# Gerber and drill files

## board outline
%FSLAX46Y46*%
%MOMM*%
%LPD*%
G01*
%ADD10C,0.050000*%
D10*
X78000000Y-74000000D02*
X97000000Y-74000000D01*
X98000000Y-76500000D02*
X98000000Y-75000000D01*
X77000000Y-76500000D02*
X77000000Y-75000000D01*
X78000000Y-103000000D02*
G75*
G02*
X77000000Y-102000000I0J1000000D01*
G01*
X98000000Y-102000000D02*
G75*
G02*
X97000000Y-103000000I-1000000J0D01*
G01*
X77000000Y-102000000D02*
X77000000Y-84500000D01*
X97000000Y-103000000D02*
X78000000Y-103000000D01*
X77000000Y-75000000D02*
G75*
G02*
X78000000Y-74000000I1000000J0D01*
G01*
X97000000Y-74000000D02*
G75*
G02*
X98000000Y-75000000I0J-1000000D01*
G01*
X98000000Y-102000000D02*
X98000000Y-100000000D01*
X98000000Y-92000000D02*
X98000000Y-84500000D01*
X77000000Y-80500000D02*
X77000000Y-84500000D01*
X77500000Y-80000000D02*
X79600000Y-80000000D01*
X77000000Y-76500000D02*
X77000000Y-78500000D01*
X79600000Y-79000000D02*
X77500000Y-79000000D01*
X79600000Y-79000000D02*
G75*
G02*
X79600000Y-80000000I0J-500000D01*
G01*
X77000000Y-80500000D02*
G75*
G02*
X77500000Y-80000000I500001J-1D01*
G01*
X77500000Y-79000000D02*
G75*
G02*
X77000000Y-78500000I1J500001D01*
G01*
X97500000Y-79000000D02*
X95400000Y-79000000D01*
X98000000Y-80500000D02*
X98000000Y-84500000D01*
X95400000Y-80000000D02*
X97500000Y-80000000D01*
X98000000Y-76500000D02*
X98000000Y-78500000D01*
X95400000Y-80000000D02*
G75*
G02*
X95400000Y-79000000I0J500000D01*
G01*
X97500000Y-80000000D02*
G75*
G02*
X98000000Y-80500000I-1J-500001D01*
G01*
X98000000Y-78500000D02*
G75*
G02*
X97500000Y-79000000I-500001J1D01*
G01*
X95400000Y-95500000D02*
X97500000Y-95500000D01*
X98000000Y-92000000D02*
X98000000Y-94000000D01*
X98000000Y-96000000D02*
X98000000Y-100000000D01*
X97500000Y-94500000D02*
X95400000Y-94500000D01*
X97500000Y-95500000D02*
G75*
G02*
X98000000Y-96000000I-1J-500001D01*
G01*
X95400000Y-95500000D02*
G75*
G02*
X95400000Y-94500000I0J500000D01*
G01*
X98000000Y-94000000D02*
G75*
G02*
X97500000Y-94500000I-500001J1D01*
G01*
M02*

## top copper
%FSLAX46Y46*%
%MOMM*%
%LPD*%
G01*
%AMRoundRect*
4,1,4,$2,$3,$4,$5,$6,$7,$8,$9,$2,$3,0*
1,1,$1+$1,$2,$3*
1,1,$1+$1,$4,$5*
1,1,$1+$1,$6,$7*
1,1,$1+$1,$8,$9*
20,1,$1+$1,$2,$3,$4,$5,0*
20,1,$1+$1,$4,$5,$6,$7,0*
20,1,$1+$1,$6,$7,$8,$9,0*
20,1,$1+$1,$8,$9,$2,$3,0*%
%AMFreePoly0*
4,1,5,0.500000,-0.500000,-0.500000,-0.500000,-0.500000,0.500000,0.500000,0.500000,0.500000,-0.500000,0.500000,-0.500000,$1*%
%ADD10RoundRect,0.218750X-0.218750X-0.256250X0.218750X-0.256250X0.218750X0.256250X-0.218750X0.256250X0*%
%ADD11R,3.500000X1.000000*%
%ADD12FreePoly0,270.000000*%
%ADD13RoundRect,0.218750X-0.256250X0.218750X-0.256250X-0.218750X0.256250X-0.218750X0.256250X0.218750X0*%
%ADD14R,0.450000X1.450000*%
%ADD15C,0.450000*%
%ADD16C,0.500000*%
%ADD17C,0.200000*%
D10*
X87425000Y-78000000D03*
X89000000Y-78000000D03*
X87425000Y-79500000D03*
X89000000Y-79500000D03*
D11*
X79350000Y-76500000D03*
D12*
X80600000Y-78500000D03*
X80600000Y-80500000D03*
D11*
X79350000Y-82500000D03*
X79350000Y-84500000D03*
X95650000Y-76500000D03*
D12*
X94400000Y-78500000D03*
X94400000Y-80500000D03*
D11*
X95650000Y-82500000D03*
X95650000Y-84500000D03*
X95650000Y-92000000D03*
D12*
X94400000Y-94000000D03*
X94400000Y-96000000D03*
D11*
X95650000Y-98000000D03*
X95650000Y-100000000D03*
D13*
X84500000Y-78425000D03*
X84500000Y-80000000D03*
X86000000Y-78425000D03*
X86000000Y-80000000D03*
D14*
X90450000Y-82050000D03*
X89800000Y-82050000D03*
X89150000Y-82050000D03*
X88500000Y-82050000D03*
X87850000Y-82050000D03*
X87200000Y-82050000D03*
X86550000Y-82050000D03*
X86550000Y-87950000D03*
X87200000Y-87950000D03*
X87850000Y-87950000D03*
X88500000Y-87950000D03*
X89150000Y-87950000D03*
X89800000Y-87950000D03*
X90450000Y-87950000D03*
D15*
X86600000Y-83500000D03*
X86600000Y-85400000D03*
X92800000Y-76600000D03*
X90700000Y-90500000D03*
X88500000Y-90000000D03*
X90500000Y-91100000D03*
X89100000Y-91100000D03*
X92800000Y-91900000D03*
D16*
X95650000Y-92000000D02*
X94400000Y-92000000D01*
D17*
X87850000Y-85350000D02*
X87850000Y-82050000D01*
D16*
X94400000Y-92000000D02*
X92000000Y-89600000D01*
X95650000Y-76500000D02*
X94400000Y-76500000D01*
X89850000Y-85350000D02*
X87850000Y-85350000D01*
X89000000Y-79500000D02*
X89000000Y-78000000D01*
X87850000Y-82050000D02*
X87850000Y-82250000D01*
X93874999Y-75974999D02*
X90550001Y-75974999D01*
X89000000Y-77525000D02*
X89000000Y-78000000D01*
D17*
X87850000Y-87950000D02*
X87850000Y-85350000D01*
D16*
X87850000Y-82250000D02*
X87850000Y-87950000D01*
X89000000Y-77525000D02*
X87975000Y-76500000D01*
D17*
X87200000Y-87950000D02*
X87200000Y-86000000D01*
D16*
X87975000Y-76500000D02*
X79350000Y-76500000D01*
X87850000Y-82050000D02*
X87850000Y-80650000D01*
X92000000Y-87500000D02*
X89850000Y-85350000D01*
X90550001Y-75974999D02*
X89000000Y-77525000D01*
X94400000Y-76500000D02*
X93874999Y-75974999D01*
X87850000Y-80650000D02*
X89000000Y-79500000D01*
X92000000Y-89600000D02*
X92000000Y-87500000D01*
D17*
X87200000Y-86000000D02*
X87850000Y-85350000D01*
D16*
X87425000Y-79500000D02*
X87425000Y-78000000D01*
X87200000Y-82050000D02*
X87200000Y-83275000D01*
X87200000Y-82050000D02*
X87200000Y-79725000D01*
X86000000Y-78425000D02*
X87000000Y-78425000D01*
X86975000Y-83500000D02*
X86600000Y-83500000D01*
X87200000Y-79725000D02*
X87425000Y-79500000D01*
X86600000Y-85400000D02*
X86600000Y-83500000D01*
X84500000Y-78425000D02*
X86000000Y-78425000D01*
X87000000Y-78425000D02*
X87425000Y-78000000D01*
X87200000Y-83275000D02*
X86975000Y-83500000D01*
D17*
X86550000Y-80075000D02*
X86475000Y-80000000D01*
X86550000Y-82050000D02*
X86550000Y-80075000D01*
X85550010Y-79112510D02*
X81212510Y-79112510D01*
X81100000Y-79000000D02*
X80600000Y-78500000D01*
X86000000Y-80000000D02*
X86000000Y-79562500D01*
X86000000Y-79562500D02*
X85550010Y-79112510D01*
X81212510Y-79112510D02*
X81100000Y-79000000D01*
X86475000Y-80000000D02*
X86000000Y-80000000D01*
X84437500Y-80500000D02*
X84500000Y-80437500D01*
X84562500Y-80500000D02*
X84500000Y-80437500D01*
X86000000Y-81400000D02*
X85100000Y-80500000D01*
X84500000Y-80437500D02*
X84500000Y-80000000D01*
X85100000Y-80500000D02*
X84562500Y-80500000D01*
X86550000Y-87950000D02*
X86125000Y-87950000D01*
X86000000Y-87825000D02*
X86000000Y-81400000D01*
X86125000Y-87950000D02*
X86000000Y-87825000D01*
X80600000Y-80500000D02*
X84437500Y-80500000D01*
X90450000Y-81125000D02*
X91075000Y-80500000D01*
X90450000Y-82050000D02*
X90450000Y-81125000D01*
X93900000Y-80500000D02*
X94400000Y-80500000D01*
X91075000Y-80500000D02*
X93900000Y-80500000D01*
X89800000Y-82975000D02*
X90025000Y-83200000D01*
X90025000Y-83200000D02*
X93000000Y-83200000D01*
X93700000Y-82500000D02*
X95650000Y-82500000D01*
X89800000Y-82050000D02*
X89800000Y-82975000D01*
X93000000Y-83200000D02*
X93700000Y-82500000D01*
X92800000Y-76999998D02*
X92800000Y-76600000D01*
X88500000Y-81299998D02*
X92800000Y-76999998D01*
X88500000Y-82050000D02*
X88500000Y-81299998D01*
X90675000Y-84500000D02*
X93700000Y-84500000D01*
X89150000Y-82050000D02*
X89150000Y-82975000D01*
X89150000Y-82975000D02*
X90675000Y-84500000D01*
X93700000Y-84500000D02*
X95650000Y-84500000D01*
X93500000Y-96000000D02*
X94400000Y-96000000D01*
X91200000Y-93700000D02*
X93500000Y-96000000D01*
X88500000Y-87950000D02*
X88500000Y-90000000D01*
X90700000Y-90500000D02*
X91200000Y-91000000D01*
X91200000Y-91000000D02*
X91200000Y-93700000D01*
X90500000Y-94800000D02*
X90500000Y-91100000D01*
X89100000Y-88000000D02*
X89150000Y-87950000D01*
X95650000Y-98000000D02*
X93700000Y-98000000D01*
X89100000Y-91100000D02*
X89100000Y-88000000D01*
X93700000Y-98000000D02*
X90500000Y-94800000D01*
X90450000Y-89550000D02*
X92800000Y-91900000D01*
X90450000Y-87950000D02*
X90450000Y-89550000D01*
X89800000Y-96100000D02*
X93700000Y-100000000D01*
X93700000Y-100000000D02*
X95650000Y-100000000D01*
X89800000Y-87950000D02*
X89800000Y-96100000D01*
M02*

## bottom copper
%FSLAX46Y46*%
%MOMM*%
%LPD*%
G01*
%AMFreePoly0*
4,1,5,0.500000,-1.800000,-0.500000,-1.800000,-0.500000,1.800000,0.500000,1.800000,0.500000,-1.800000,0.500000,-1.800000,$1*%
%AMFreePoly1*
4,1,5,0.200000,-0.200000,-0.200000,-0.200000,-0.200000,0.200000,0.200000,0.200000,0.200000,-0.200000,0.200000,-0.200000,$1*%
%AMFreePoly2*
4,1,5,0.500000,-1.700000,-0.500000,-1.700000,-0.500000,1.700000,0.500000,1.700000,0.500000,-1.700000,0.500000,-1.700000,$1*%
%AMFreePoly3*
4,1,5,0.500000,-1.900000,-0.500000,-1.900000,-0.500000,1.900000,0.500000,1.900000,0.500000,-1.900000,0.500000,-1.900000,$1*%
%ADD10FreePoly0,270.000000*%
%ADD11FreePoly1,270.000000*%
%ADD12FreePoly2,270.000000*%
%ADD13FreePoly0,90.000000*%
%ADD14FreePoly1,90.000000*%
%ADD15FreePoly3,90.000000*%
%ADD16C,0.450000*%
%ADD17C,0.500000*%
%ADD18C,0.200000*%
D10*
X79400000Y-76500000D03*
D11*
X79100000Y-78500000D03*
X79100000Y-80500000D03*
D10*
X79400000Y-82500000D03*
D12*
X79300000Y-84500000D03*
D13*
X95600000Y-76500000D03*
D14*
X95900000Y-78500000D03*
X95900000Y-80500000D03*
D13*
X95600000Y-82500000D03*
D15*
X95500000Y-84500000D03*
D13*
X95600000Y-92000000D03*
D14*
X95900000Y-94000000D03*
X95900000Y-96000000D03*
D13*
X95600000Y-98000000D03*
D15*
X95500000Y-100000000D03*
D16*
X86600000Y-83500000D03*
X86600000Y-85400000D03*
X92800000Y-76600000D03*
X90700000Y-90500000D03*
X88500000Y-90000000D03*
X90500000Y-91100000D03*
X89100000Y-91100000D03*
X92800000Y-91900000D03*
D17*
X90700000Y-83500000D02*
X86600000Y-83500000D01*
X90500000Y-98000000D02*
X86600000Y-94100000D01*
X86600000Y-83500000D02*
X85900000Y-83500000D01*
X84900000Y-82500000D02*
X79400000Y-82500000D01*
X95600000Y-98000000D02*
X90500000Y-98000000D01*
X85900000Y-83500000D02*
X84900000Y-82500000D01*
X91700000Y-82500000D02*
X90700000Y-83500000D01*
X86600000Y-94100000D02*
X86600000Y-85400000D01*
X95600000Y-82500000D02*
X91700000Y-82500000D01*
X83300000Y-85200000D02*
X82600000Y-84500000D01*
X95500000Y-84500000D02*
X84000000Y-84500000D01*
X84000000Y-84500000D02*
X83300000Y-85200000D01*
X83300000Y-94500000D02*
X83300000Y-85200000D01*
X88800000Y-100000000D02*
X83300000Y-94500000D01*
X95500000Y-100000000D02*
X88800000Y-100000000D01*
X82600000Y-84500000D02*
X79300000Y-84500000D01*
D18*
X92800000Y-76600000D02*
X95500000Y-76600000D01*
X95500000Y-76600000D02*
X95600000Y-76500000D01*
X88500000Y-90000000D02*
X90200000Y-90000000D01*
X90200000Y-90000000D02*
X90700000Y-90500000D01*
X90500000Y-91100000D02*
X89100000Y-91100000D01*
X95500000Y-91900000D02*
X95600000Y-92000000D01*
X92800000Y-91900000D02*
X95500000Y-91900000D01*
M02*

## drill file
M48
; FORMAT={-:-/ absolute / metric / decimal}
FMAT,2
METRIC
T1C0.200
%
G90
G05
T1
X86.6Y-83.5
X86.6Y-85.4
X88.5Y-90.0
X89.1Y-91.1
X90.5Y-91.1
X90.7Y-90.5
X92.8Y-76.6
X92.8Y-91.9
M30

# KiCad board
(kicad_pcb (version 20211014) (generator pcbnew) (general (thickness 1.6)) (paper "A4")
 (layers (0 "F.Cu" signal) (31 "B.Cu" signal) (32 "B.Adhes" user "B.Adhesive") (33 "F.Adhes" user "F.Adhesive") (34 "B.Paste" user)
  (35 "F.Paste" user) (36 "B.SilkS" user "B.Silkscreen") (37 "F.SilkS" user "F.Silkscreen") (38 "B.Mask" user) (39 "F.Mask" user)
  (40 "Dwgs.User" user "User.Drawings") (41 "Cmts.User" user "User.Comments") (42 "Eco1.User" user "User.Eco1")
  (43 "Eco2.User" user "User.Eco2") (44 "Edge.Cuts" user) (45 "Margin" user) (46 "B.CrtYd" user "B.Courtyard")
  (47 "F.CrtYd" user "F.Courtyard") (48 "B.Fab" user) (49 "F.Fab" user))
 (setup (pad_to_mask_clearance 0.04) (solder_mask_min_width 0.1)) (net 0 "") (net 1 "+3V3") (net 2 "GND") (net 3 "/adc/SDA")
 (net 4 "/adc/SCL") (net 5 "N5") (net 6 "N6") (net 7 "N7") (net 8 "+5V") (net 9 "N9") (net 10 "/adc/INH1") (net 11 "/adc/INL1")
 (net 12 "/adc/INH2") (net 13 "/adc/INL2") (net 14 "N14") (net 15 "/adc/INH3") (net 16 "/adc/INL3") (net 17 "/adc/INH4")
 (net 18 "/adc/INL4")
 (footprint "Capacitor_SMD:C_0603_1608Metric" (layer "F.Cu") (at 88.2125 78)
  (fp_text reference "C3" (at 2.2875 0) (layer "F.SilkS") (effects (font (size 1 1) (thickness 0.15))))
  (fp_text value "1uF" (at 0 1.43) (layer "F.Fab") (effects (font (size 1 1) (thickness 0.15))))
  (pad "1" smd roundrect locked (at -0.7875 0) (size 0.875 0.95) (layers "F.Cu" "F.Paste" "F.Mask") (roundrect_rratio 0.25) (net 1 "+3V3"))
  (pad "2" smd roundrect locked (at 0.7875 0) (size 0.875 0.95) (layers "F.Cu" "F.Paste" "F.Mask") (roundrect_rratio 0.25) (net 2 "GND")))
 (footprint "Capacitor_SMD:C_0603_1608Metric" (layer "F.Cu") (at 88.2125 79.5)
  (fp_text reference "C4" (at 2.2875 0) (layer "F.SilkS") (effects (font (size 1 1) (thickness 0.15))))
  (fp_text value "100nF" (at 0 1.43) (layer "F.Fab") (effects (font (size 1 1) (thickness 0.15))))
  (pad "1" smd roundrect locked (at -0.7875 0) (size 0.875 0.95) (layers "F.Cu" "F.Paste" "F.Mask") (roundrect_rratio 0.25) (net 1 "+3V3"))
  (pad "2" smd roundrect locked (at 0.7875 0) (size 0.875 0.95) (layers "F.Cu" "F.Paste" "F.Mask") (roundrect_rratio 0.25) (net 2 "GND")))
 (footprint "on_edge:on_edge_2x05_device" (layer "F.Cu") (at 77 80.5 -90)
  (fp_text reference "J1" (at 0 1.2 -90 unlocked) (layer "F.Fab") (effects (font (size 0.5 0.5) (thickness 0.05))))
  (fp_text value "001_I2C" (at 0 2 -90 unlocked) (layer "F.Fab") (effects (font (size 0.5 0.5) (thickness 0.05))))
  (fp_line (start 0 0) (end 4 0) (layer "Edge.Cuts") (width 0.05))
  (fp_line (start -0.5 -0.5) (end -0.5 -2.6) (layer "Edge.Cuts") (width 0.05))
  (fp_line (start -4 0) (end -2 0) (layer "Edge.Cuts") (width 0.05))
  (fp_line (start -1.5 -2.6) (end -1.5 -0.5) (layer "Edge.Cuts") (width 0.05))
  (fp_arc (start -1.5 -2.6) (mid -1 -3.1) (end -0.5 -2.6) (layer "Edge.Cuts") (width 0.05))
  (fp_arc (start 0 0) (mid -0.353553 -0.146447) (end -0.5 -0.5) (layer "Edge.Cuts") (width 0.05))
  (fp_arc (start -1.5 -0.5) (mid -1.646447 -0.146447) (end -2 0) (layer "Edge.Cuts") (width 0.05))
  (pad "1" smd rect locked (at -4 -2.35 90) (size 1 3.5) (layers "F.Cu" "F.Mask") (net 2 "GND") (zone_connect 0))
  (pad "2" smd custom locked (at -2 -3.6 270) (size 1 1) (layers "F.Cu" "F.Mask") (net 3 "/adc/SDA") (zone_connect 0)
   (options (clearance outline) (anchor rect)) (primitives))
  (pad "3" smd custom locked (at 0 -3.6 270) (size 1 1) (layers "F.Cu" "F.Mask") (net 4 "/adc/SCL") (zone_connect 0)
   (options (clearance outline) (anchor rect)) (primitives))
  (pad "4" smd rect locked (at 2 -2.35 90) (size 1 3.5) (layers "F.Cu" "F.Mask") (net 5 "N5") (zone_connect 0))
  (pad "5" smd rect locked (at 4 -2.35 90) (size 1 3.5) (layers "F.Cu" "F.Mask") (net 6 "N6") (zone_connect 0))
  (pad "6" smd custom locked (at -4 -2.4 270) (size 1 3.6) (layers "B.Cu" "B.Mask") (zone_connect 0)
   (options (clearance outline) (anchor rect)) (primitives))
  (pad "7" smd custom locked (at -2 -2.1 270) (size 0.4 0.4) (layers "B.Cu" "B.Mask") (zone_connect 0)
   (options (clearance outline) (anchor rect)) (primitives))
  (pad "8" smd custom locked (at 0 -2.1 270) (size 0.4 0.4) (layers "B.Cu" "B.Mask") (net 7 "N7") (zone_connect 0)
   (options (clearance outline) (anchor rect)) (primitives))
  (pad "9" smd custom locked (at 2 -2.4 270) (size 1 3.6) (layers "B.Cu" "B.Mask") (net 1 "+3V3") (zone_connect 0)
   (options (clearance outline) (anchor rect)) (primitives))
  (pad "10" smd custom locked (at 4 -2.3 270) (size 1 3.4) (layers "B.Cu" "B.Mask") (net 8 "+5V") (zone_connect 0)
   (options (clearance outline) (anchor rect)) (primitives)))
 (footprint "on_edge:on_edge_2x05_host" (layer "F.Cu") (at 98 80.5 -90)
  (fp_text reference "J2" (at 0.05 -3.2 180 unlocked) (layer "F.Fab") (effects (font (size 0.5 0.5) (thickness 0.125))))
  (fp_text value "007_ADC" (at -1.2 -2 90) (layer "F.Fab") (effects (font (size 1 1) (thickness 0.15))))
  (fp_line (start -1.5 0.5) (end -1.5 2.6) (layer "Edge.Cuts") (width 0.05))
  (fp_line (start 0 0) (end 4 0) (layer "Edge.Cuts") (width 0.05))
  (fp_line (start -0.5 2.6) (end -0.5 0.5) (layer "Edge.Cuts") (width 0.05))
  (fp_line (start -4 0) (end -2 0) (layer "Edge.Cuts") (width 0.05))
  (fp_arc (start -0.5 2.6) (mid -1 3.1) (end -1.5 2.6) (layer "Edge.Cuts") (width 0.05))
  (fp_arc (start -0.5 0.5) (mid -0.353553 0.146447) (end 0 0) (layer "Edge.Cuts") (width 0.05))
  (fp_arc (start -2 0) (mid -1.646447 0.146447) (end -1.5 0.5) (layer "Edge.Cuts") (width 0.05))
  (pad "1" smd rect locked (at -4 2.35 270) (size 1 3.5) (layers "F.Cu" "F.Mask") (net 2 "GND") (zone_connect 0))
  (pad "2" smd custom locked (at -2 3.6 270) (size 1 1) (layers "F.Cu" "F.Mask") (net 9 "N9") (zone_connect 0)
   (options (clearance outline) (anchor rect)) (primitives))
  (pad "3" smd custom locked (at 0 3.6 270) (size 1 1) (layers "F.Cu" "F.Mask") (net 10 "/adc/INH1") (zone_connect 0)
   (options (clearance outline) (anchor rect)) (primitives))
  (pad "4" smd rect locked (at 2 2.35 270) (size 1 3.5) (layers "F.Cu" "F.Mask") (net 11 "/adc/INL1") (zone_connect 0))
  (pad "5" smd rect locked (at 4 2.35 270) (size 1 3.5) (layers "F.Cu" "F.Mask") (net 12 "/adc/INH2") (zone_connect 0))
  (pad "6" smd custom locked (at -4 2.4 90) (size 1 3.6) (layers "B.Cu" "B.Mask") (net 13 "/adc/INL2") (zone_connect 0)
   (options (clearance outline) (anchor rect)) (primitives))
  (pad "7" smd custom locked (at -2 2.1 90) (size 0.4 0.4) (layers "B.Cu" "B.Mask") (zone_connect 0)
   (options (clearance outline) (anchor rect)) (primitives))
  (pad "8" smd custom locked (at 0 2.1 90) (size 0.4 0.4) (layers "B.Cu" "B.Mask") (zone_connect 0)
   (options (clearance outline) (anchor rect)) (primitives))
  (pad "9" smd custom locked (at 2 2.4 90) (size 1 3.6) (layers "B.Cu" "B.Mask") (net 1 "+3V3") (zone_connect 0)
   (options (clearance outline) (anchor rect)) (primitives))
  (pad "10" smd custom locked (at 4 2.5 90) (size 1 3.8) (layers "B.Cu" "B.Mask") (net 8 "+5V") (zone_connect 0)
   (options (clearance outline) (anchor rect)) (primitives)))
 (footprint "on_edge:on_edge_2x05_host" (layer "F.Cu") (at 98 96 -90)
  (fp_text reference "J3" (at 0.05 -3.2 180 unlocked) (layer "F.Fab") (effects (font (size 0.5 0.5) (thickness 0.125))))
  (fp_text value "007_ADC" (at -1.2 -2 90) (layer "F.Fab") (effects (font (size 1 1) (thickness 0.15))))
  (fp_line (start -0.5 2.6) (end -0.5 0.5) (layer "Edge.Cuts") (width 0.05))
  (fp_line (start -4 0) (end -2 0) (layer "Edge.Cuts") (width 0.05))
  (fp_line (start 0 0) (end 4 0) (layer "Edge.Cuts") (width 0.05))
  (fp_line (start -1.5 0.5) (end -1.5 2.6) (layer "Edge.Cuts") (width 0.05))
  (fp_arc (start -0.5 0.5) (mid -0.353553 0.146447) (end 0 0) (layer "Edge.Cuts") (width 0.05))
  (fp_arc (start -0.5 2.6) (mid -1 3.1) (end -1.5 2.6) (layer "Edge.Cuts") (width 0.05))
  (fp_arc (start -2 0) (mid -1.646447 0.146447) (end -1.5 0.5) (layer "Edge.Cuts") (width 0.05))
  (pad "1" smd rect locked (at -4 2.35 270) (size 1 3.5) (layers "F.Cu" "F.Mask") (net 2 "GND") (zone_connect 0))
  (pad "2" smd custom locked (at -2 3.6 270) (size 1 1) (layers "F.Cu" "F.Mask") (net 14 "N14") (zone_connect 0)
   (options (clearance outline) (anchor rect)) (primitives))
  (pad "3" smd custom locked (at 0 3.6 270) (size 1 1) (layers "F.Cu" "F.Mask") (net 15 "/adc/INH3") (zone_connect 0)
   (options (clearance outline) (anchor rect)) (primitives))
  (pad "4" smd rect locked (at 2 2.35 270) (size 1 3.5) (layers "F.Cu" "F.Mask") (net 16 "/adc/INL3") (zone_connect 0))
  (pad "5" smd rect locked (at 4 2.35 270) (size 1 3.5) (layers "F.Cu" "F.Mask") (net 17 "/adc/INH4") (zone_connect 0))
  (pad "6" smd custom locked (at -4 2.4 90) (size 1 3.6) (layers "B.Cu" "B.Mask") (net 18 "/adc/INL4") (zone_connect 0)
   (options (clearance outline) (anchor rect)) (primitives))
  (pad "7" smd custom locked (at -2 2.1 90) (size 0.4 0.4) (layers "B.Cu" "B.Mask") (zone_connect 0)
   (options (clearance outline) (anchor rect)) (primitives))
  (pad "8" smd custom locked (at 0 2.1 90) (size 0.4 0.4) (layers "B.Cu" "B.Mask") (zone_connect 0)
   (options (clearance outline) (anchor rect)) (primitives))
  (pad "9" smd custom locked (at 2 2.4 90) (size 1 3.6) (layers "B.Cu" "B.Mask") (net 1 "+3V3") (zone_connect 0)
   (options (clearance outline) (anchor rect)) (primitives))
  (pad "10" smd custom locked (at 4 2.5 90) (size 1 3.8) (layers "B.Cu" "B.Mask") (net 8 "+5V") (zone_connect 0)
   (options (clearance outline) (anchor rect)) (primitives)))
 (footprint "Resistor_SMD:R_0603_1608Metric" (layer "F.Cu") (at 84.5 79.2125 -90)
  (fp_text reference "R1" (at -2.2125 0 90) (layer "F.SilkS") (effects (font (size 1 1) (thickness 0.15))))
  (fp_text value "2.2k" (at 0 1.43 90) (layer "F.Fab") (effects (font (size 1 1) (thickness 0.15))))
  (pad "1" smd roundrect locked (at -0.7875 0 270) (size 0.875 0.95) (layers "F.Cu" "F.Paste" "F.Mask") (roundrect_rratio 0.25)
   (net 1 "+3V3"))
  (pad "2" smd roundrect locked (at 0.7875 0 270) (size 0.875 0.95) (layers "F.Cu" "F.Paste" "F.Mask") (roundrect_rratio 0.25)
   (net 4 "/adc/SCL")))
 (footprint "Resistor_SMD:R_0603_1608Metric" (layer "F.Cu") (at 86 79.2125 -90)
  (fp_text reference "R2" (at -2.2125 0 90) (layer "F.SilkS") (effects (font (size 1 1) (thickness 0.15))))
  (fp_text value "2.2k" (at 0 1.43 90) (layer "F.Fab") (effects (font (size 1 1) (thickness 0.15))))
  (pad "1" smd roundrect locked (at -0.7875 0 270) (size 0.875 0.95) (layers "F.Cu" "F.Paste" "F.Mask") (roundrect_rratio 0.25)
   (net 1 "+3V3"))
  (pad "2" smd roundrect locked (at 0.7875 0 270) (size 0.875 0.95) (layers "F.Cu" "F.Paste" "F.Mask") (roundrect_rratio 0.25)
   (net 3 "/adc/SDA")))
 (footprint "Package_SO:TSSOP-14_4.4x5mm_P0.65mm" (layer "F.Cu") (at 88.5 85 -90)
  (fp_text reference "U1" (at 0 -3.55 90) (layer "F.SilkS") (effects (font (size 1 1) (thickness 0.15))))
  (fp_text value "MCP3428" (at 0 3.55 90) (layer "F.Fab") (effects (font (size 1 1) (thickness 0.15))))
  (pad "1" smd rect locked (at -2.95 -1.95 270) (size 1.45 0.45) (layers "F.Cu" "F.Paste" "F.Mask") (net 10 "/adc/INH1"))
  (pad "2" smd rect locked (at -2.95 -1.3 270) (size 1.45 0.45) (layers "F.Cu" "F.Paste" "F.Mask") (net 11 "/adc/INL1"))
  (pad "3" smd rect locked (at -2.95 -0.65 270) (size 1.45 0.45) (layers "F.Cu" "F.Paste" "F.Mask") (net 12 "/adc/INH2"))
  (pad "4" smd rect locked (at -2.95 0 270) (size 1.45 0.45) (layers "F.Cu" "F.Paste" "F.Mask") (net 13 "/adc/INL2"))
  (pad "5" smd rect locked (at -2.95 0.65 270) (size 1.45 0.45) (layers "F.Cu" "F.Paste" "F.Mask") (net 2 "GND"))
  (pad "6" smd rect locked (at -2.95 1.3 270) (size 1.45 0.45) (layers "F.Cu" "F.Paste" "F.Mask") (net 1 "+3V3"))
  (pad "7" smd rect locked (at -2.95 1.95 270) (size 1.45 0.45) (layers "F.Cu" "F.Paste" "F.Mask") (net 3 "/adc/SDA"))
  (pad "8" smd rect locked (at 2.95 1.95 270) (size 1.45 0.45) (layers "F.Cu" "F.Paste" "F.Mask") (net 4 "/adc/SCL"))
  (pad "9" smd rect locked (at 2.95 1.3 270) (size 1.45 0.45) (layers "F.Cu" "F.Paste" "F.Mask") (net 2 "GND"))
  (pad "10" smd rect locked (at 2.95 0.65 270) (size 1.45 0.45) (layers "F.Cu" "F.Paste" "F.Mask") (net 2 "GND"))
  (pad "11" smd rect locked (at 2.95 0 270) (size 1.45 0.45) (layers "F.Cu" "F.Paste" "F.Mask") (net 15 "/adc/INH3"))
  (pad "12" smd rect locked (at 2.95 -0.65 270) (size 1.45 0.45) (layers "F.Cu" "F.Paste" "F.Mask") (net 16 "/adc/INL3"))
  (pad "13" smd rect locked (at 2.95 -1.3 270) (size 1.45 0.45) (layers "F.Cu" "F.Paste" "F.Mask") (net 17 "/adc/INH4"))
  (pad "14" smd rect locked (at 2.95 -1.95 270) (size 1.45 0.45) (layers "F.Cu" "F.Paste" "F.Mask") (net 18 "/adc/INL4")))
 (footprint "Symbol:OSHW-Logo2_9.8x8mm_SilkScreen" (layer "F.Cu") (at 82.6 93.6)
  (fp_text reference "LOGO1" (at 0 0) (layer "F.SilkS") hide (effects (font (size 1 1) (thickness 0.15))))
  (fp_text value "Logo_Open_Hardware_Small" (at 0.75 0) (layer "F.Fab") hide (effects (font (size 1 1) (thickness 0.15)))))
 (gr_line (start 78 74) (end 97 74) (layer "Edge.Cuts") (width 0.05))
 (gr_line (start 98 76.5) (end 98 75) (layer "Edge.Cuts") (width 0.05))
 (gr_line (start 77 76.5) (end 77 75) (layer "Edge.Cuts") (width 0.05))
 (gr_arc (start 78 103) (mid 77.292893 102.707107) (end 77 102) (layer "Edge.Cuts") (width 0.05))
 (gr_arc (start 98 102) (mid 97.707107 102.707107) (end 97 103) (layer "Edge.Cuts") (width 0.05))
 (gr_line (start 77 102) (end 77 84.5) (layer "Edge.Cuts") (width 0.05))
 (gr_line (start 97 103) (end 78 103) (layer "Edge.Cuts") (width 0.05))
 (gr_arc (start 77 75) (mid 77.292893 74.292893) (end 78 74) (layer "Edge.Cuts") (width 0.05))
 (gr_arc (start 97 74) (mid 97.707107 74.292893) (end 98 75) (layer "Edge.Cuts") (width 0.05))
 (gr_line (start 98 102) (end 98 100) (layer "Edge.Cuts") (width 0.05))
 (gr_line (start 98 92) (end 98 84.5) (layer "Edge.Cuts") (width 0.05))
 (segment (start 95.65 92) (end 94.4 92) (width 0.5) (layer "F.Cu") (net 2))
 (segment (start 87.85 85.35) (end 87.85 82.05) (width 0.2) (layer "F.Cu") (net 2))
 (segment (start 94.4 92) (end 92 89.6) (width 0.5) (layer "F.Cu") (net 2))
 (segment (start 95.65 76.5) (end 94.4 76.5) (width 0.5) (layer "F.Cu") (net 2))
 (segment (start 89.85 85.35) (end 87.85 85.35) (width 0.5) (layer "F.Cu") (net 2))
 (segment (start 89 79.5) (end 89 78) (width 0.5) (layer "F.Cu") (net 2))
 (segment (start 87.85 82.05) (end 87.85 82.25) (width 0.5) (layer "F.Cu") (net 2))
 (segment (start 93.874999 75.974999) (end 90.550001 75.974999) (width 0.5) (layer "F.Cu") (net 2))
 (segment (start 89 77.525) (end 89 78) (width 0.5) (layer "F.Cu") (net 2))
 (segment (start 87.85 87.95) (end 87.85 85.35) (width 0.2) (layer "F.Cu") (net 2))
 (segment (start 87.85 82.25) (end 87.85 87.95) (width 0.5) (layer "F.Cu") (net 2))
 (segment (start 89 77.525) (end 87.975 76.5) (width 0.5) (layer "F.Cu") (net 2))
 (segment (start 87.2 87.95) (end 87.2 86) (width 0.2) (layer "F.Cu") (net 2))
 (segment (start 87.975 76.5) (end 79.35 76.5) (width 0.5) (layer "F.Cu") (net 2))
 (segment (start 87.85 82.05) (end 87.85 80.65) (width 0.5) (layer "F.Cu") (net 2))
 (segment (start 92 87.5) (end 89.85 85.35) (width 0.5) (layer "F.Cu") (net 2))
 (segment (start 90.550001 75.974999) (end 89 77.525) (width 0.5) (layer "F.Cu") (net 2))
 (segment (start 94.4 76.5) (end 93.874999 75.974999) (width 0.5) (layer "F.Cu") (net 2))
 (segment (start 87.85 80.65) (end 89 79.5) (width 0.5) (layer "F.Cu") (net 2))
 (segment (start 92 89.6) (end 92 87.5) (width 0.5) (layer "F.Cu") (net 2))
 (segment (start 87.2 86) (end 87.85 85.35) (width 0.2) (layer "F.Cu") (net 2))
 (segment (start 87.425 79.5) (end 87.425 78) (width 0.5) (layer "F.Cu") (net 1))
 (segment (start 87.2 82.05) (end 87.2 83.275) (width 0.5) (layer "F.Cu") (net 1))
 (segment (start 87.2 82.05) (end 87.2 79.725) (width 0.5) (layer "F.Cu") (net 1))
 (segment (start 86 78.425) (end 87 78.425) (width 0.5) (layer "F.Cu") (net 1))
 (segment (start 86.975 83.5) (end 86.6 83.5) (width 0.5) (layer "F.Cu") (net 1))
 (segment (start 87.2 79.725) (end 87.425 79.5) (width 0.5) (layer "F.Cu") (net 1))
 (segment (start 86.6 85.4) (end 86.6 83.5) (width 0.5) (layer "F.Cu") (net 1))
 (segment (start 84.5 78.425) (end 86 78.425) (width 0.5) (layer "F.Cu") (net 1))
 (segment (start 87 78.425) (end 87.425 78) (width 0.5) (layer "F.Cu") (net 1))
 (segment (start 87.2 83.275) (end 86.975 83.5) (width 0.5) (layer "F.Cu") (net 1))
 (via (at 86.6 83.5) (size 0.45) (drill 0.2) (layers "F.Cu" "B.Cu") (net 1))
 (via (at 86.6 85.4) (size 0.45) (drill 0.2) (layers "F.Cu" "B.Cu") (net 1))
 (segment (start 90.7 83.5) (end 86.6 83.5) (width 0.5) (layer "B.Cu") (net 1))
 (segment (start 90.5 98) (end 86.6 94.1) (width 0.5) (layer "B.Cu") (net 1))
 (segment (start 86.6 83.5) (end 85.9 83.5) (width 0.5) (layer "B.Cu") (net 1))
 (segment (start 84.9 82.5) (end 79.4 82.5) (width 0.5) (layer "B.Cu") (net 1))
 (segment (start 95.6 98) (end 90.5 98) (width 0.5) (layer "B.Cu") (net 1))
 (segment (start 85.9 83.5) (end 84.9 82.5) (width 0.5) (layer "B.Cu") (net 1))
 (segment (start 91.7 82.5) (end 90.7 83.5) (width 0.5) (layer "B.Cu") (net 1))
 (segment (start 86.6 94.1) (end 86.6 85.4) (width 0.5) (layer "B.Cu") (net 1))
 (segment (start 95.6 82.5) (end 91.7 82.5) (width 0.5) (layer "B.Cu") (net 1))
 (segment (start 83.3 85.2) (end 82.6 84.5) (width 0.5) (layer "B.Cu") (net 8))
 (segment (start 95.5 84.5) (end 84 84.5) (width 0.5) (layer "B.Cu") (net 8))
 (segment (start 84 84.5) (end 83.3 85.2) (width 0.5) (layer "B.Cu") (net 8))
 (segment (start 83.3 94.5) (end 83.3 85.2) (width 0.5) (layer "B.Cu") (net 8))
 (segment (start 88.8 100) (end 83.3 94.5) (width 0.5) (layer "B.Cu") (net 8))
 (segment (start 95.5 100) (end 88.8 100) (width 0.5) (layer "B.Cu") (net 8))
 (segment (start 82.6 84.5) (end 79.3 84.5) (width 0.5) (layer "B.Cu") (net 8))
 (segment (start 86.55 80.075) (end 86.475 80) (width 0.2) (layer "F.Cu") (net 3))
 (segment (start 86.55 82.05) (end 86.55 80.075) (width 0.2) (layer "F.Cu") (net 3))
 (segment (start 85.55001 79.11251) (end 81.21251 79.11251) (width 0.2) (layer "F.Cu") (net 3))
 (segment (start 81.1 79) (end 80.6 78.5) (width 0.2) (layer "F.Cu") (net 3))
 (segment (start 86 80) (end 86 79.5625) (width 0.2) (layer "F.Cu") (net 3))
 (segment (start 86 79.5625) (end 85.55001 79.11251) (width 0.2) (layer "F.Cu") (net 3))
 (segment (start 81.21251 79.11251) (end 81.1 79) (width 0.2) (layer "F.Cu") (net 3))
 (segment (start 86.475 80) (end 86 80) (width 0.2) (layer "F.Cu") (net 3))
 (segment (start 84.4375 80.5) (end 84.5 80.4375) (width 0.2) (layer "F.Cu") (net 4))
 (segment (start 84.5625 80.5) (end 84.5 80.4375) (width 0.2) (layer "F.Cu") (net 4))
 (segment (start 86 81.4) (end 85.1 80.5) (width 0.2) (layer "F.Cu") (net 4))
 (segment (start 84.5 80.4375) (end 84.5 80) (width 0.2) (layer "F.Cu") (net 4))
 (segment (start 85.1 80.5) (end 84.5625 80.5) (width 0.2) (layer "F.Cu") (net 4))
 (segment (start 86.55 87.95) (end 86.125 87.95) (width 0.2) (layer "F.Cu") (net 4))
 (segment (start 86 87.825) (end 86 81.4) (width 0.2) (layer "F.Cu") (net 4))
 (segment (start 86.125 87.95) (end 86 87.825) (width 0.2) (layer "F.Cu") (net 4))
 (segment (start 80.6 80.5) (end 84.4375 80.5) (width 0.2) (layer "F.Cu") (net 4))
 (segment (start 90.45 81.125) (end 91.075 80.5) (width 0.2) (layer "F.Cu") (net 10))
 (segment (start 90.45 82.05) (end 90.45 81.125) (width 0.2) (layer "F.Cu") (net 10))
 (segment (start 93.9 80.5) (end 94.4 80.5) (width 0.2) (layer "F.Cu") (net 10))
 (segment (start 91.075 80.5) (end 93.9 80.5) (width 0.2) (layer "F.Cu") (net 10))
 (segment (start 89.8 82.975) (end 90.025 83.2) (width 0.2) (layer "F.Cu") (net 11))
 (segment (start 90.025 83.2) (end 93 83.2) (width 0.2) (layer "F.Cu") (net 11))
 (segment (start 93.7 82.5) (end 95.65 82.5) (width 0.2) (layer "F.Cu") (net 11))
 (segment (start 89.8 82.05) (end 89.8 82.975) (width 0.2) (layer "F.Cu") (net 11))
 (segment (start 93 83.2) (end 93.7 82.5) (width 0.2) (layer "F.Cu") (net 11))
 (segment (start 92.8 76.999998) (end 92.8 76.6) (width 0.2) (layer "F.Cu") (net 13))
 (segment (start 88.5 81.299998) (end 92.8 76.999998) (width 0.2) (layer "F.Cu") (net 13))
 (segment (start 88.5 82.05) (end 88.5 81.299998) (width 0.2) (layer "F.Cu") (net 13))
 (via (at 92.8 76.6) (size 0.45) (drill 0.2) (layers "F.Cu" "B.Cu") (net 13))
 (segment (start 92.8 76.6) (end 95.5 76.6) (width 0.2) (layer "B.Cu") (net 13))
 (segment (start 95.5 76.6) (end 95.6 76.5) (width 0.2) (layer "B.Cu") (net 13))
 (segment (start 90.675 84.5) (end 93.7 84.5) (width 0.2) (layer "F.Cu") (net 12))
 (segment (start 89.15 82.05) (end 89.15 82.975) (width 0.2) (layer "F.Cu") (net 12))
 (segment (start 89.15 82.975) (end 90.675 84.5) (width 0.2) (layer "F.Cu") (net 12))
 (segment (start 93.7 84.5) (end 95.65 84.5) (width 0.2) (layer "F.Cu") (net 12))
 (segment (start 93.5 96) (end 94.4 96) (width 0.2) (layer "F.Cu") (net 15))
 (segment (start 91.2 93.7) (end 93.5 96) (width 0.2) (layer "F.Cu") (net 15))
 (segment (start 88.5 87.95) (end 88.5 90) (width 0.2) (layer "F.Cu") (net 15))
 (segment (start 90.7 90.5) (end 91.2 91) (width 0.2) (layer "F.Cu") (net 15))
 (segment (start 91.2 91) (end 91.2 93.7) (width 0.2) (layer "F.Cu") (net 15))
 (via (at 90.7 90.5) (size 0.45) (drill 0.2) (layers "F.Cu" "B.Cu") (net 15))
 (via (at 88.5 90) (size 0.45) (drill 0.2) (layers "F.Cu" "B.Cu") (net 15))
 (segment (start 88.5 90) (end 90.2 90) (width 0.2) (layer "B.Cu") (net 15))
 (segment (start 90.2 90) (end 90.7 90.5) (width 0.2) (layer "B.Cu") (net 15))
 (segment (start 90.5 94.8) (end 90.5 91.1) (width 0.2) (layer "F.Cu") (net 16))
 (segment (start 89.1 88) (end 89.15 87.95) (width 0.2) (layer "F.Cu") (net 16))
 (segment (start 95.65 98) (end 93.7 98) (width 0.2) (layer "F.Cu") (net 16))
 (segment (start 89.1 91.1) (end 89.1 88) (width 0.2) (layer "F.Cu") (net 16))
 (segment (start 93.7 98) (end 90.5 94.8) (width 0.2) (layer "F.Cu") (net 16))
 (via (at 90.5 91.1) (size 0.45) (drill 0.2) (layers "F.Cu" "B.Cu") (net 16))
 (via (at 89.1 91.1) (size 0.45) (drill 0.2) (layers "F.Cu" "B.Cu") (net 16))
 (segment (start 90.5 91.1) (end 89.1 91.1) (width 0.2) (layer "B.Cu") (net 16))
 (segment (start 90.45 89.55) (end 92.8 91.9) (width 0.2) (layer "F.Cu") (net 18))
 (segment (start 90.45 87.95) (end 90.45 89.55) (width 0.2) (layer "F.Cu") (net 18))
 (via (at 92.8 91.9) (size 0.45) (drill 0.2) (layers "F.Cu" "B.Cu") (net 18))
 (segment (start 95.5 91.9) (end 95.6 92) (width 0.2) (layer "B.Cu") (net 18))
 (segment (start 92.8 91.9) (end 95.5 91.9) (width 0.2) (layer "B.Cu") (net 18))
 (segment (start 89.8 96.1) (end 93.7 100) (width 0.2) (layer "F.Cu") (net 17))
 (segment (start 93.7 100) (end 95.65 100) (width 0.2) (layer "F.Cu") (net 17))
 (segment (start 89.8 87.95) (end 89.8 96.1) (width 0.2) (layer "F.Cu") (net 17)))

